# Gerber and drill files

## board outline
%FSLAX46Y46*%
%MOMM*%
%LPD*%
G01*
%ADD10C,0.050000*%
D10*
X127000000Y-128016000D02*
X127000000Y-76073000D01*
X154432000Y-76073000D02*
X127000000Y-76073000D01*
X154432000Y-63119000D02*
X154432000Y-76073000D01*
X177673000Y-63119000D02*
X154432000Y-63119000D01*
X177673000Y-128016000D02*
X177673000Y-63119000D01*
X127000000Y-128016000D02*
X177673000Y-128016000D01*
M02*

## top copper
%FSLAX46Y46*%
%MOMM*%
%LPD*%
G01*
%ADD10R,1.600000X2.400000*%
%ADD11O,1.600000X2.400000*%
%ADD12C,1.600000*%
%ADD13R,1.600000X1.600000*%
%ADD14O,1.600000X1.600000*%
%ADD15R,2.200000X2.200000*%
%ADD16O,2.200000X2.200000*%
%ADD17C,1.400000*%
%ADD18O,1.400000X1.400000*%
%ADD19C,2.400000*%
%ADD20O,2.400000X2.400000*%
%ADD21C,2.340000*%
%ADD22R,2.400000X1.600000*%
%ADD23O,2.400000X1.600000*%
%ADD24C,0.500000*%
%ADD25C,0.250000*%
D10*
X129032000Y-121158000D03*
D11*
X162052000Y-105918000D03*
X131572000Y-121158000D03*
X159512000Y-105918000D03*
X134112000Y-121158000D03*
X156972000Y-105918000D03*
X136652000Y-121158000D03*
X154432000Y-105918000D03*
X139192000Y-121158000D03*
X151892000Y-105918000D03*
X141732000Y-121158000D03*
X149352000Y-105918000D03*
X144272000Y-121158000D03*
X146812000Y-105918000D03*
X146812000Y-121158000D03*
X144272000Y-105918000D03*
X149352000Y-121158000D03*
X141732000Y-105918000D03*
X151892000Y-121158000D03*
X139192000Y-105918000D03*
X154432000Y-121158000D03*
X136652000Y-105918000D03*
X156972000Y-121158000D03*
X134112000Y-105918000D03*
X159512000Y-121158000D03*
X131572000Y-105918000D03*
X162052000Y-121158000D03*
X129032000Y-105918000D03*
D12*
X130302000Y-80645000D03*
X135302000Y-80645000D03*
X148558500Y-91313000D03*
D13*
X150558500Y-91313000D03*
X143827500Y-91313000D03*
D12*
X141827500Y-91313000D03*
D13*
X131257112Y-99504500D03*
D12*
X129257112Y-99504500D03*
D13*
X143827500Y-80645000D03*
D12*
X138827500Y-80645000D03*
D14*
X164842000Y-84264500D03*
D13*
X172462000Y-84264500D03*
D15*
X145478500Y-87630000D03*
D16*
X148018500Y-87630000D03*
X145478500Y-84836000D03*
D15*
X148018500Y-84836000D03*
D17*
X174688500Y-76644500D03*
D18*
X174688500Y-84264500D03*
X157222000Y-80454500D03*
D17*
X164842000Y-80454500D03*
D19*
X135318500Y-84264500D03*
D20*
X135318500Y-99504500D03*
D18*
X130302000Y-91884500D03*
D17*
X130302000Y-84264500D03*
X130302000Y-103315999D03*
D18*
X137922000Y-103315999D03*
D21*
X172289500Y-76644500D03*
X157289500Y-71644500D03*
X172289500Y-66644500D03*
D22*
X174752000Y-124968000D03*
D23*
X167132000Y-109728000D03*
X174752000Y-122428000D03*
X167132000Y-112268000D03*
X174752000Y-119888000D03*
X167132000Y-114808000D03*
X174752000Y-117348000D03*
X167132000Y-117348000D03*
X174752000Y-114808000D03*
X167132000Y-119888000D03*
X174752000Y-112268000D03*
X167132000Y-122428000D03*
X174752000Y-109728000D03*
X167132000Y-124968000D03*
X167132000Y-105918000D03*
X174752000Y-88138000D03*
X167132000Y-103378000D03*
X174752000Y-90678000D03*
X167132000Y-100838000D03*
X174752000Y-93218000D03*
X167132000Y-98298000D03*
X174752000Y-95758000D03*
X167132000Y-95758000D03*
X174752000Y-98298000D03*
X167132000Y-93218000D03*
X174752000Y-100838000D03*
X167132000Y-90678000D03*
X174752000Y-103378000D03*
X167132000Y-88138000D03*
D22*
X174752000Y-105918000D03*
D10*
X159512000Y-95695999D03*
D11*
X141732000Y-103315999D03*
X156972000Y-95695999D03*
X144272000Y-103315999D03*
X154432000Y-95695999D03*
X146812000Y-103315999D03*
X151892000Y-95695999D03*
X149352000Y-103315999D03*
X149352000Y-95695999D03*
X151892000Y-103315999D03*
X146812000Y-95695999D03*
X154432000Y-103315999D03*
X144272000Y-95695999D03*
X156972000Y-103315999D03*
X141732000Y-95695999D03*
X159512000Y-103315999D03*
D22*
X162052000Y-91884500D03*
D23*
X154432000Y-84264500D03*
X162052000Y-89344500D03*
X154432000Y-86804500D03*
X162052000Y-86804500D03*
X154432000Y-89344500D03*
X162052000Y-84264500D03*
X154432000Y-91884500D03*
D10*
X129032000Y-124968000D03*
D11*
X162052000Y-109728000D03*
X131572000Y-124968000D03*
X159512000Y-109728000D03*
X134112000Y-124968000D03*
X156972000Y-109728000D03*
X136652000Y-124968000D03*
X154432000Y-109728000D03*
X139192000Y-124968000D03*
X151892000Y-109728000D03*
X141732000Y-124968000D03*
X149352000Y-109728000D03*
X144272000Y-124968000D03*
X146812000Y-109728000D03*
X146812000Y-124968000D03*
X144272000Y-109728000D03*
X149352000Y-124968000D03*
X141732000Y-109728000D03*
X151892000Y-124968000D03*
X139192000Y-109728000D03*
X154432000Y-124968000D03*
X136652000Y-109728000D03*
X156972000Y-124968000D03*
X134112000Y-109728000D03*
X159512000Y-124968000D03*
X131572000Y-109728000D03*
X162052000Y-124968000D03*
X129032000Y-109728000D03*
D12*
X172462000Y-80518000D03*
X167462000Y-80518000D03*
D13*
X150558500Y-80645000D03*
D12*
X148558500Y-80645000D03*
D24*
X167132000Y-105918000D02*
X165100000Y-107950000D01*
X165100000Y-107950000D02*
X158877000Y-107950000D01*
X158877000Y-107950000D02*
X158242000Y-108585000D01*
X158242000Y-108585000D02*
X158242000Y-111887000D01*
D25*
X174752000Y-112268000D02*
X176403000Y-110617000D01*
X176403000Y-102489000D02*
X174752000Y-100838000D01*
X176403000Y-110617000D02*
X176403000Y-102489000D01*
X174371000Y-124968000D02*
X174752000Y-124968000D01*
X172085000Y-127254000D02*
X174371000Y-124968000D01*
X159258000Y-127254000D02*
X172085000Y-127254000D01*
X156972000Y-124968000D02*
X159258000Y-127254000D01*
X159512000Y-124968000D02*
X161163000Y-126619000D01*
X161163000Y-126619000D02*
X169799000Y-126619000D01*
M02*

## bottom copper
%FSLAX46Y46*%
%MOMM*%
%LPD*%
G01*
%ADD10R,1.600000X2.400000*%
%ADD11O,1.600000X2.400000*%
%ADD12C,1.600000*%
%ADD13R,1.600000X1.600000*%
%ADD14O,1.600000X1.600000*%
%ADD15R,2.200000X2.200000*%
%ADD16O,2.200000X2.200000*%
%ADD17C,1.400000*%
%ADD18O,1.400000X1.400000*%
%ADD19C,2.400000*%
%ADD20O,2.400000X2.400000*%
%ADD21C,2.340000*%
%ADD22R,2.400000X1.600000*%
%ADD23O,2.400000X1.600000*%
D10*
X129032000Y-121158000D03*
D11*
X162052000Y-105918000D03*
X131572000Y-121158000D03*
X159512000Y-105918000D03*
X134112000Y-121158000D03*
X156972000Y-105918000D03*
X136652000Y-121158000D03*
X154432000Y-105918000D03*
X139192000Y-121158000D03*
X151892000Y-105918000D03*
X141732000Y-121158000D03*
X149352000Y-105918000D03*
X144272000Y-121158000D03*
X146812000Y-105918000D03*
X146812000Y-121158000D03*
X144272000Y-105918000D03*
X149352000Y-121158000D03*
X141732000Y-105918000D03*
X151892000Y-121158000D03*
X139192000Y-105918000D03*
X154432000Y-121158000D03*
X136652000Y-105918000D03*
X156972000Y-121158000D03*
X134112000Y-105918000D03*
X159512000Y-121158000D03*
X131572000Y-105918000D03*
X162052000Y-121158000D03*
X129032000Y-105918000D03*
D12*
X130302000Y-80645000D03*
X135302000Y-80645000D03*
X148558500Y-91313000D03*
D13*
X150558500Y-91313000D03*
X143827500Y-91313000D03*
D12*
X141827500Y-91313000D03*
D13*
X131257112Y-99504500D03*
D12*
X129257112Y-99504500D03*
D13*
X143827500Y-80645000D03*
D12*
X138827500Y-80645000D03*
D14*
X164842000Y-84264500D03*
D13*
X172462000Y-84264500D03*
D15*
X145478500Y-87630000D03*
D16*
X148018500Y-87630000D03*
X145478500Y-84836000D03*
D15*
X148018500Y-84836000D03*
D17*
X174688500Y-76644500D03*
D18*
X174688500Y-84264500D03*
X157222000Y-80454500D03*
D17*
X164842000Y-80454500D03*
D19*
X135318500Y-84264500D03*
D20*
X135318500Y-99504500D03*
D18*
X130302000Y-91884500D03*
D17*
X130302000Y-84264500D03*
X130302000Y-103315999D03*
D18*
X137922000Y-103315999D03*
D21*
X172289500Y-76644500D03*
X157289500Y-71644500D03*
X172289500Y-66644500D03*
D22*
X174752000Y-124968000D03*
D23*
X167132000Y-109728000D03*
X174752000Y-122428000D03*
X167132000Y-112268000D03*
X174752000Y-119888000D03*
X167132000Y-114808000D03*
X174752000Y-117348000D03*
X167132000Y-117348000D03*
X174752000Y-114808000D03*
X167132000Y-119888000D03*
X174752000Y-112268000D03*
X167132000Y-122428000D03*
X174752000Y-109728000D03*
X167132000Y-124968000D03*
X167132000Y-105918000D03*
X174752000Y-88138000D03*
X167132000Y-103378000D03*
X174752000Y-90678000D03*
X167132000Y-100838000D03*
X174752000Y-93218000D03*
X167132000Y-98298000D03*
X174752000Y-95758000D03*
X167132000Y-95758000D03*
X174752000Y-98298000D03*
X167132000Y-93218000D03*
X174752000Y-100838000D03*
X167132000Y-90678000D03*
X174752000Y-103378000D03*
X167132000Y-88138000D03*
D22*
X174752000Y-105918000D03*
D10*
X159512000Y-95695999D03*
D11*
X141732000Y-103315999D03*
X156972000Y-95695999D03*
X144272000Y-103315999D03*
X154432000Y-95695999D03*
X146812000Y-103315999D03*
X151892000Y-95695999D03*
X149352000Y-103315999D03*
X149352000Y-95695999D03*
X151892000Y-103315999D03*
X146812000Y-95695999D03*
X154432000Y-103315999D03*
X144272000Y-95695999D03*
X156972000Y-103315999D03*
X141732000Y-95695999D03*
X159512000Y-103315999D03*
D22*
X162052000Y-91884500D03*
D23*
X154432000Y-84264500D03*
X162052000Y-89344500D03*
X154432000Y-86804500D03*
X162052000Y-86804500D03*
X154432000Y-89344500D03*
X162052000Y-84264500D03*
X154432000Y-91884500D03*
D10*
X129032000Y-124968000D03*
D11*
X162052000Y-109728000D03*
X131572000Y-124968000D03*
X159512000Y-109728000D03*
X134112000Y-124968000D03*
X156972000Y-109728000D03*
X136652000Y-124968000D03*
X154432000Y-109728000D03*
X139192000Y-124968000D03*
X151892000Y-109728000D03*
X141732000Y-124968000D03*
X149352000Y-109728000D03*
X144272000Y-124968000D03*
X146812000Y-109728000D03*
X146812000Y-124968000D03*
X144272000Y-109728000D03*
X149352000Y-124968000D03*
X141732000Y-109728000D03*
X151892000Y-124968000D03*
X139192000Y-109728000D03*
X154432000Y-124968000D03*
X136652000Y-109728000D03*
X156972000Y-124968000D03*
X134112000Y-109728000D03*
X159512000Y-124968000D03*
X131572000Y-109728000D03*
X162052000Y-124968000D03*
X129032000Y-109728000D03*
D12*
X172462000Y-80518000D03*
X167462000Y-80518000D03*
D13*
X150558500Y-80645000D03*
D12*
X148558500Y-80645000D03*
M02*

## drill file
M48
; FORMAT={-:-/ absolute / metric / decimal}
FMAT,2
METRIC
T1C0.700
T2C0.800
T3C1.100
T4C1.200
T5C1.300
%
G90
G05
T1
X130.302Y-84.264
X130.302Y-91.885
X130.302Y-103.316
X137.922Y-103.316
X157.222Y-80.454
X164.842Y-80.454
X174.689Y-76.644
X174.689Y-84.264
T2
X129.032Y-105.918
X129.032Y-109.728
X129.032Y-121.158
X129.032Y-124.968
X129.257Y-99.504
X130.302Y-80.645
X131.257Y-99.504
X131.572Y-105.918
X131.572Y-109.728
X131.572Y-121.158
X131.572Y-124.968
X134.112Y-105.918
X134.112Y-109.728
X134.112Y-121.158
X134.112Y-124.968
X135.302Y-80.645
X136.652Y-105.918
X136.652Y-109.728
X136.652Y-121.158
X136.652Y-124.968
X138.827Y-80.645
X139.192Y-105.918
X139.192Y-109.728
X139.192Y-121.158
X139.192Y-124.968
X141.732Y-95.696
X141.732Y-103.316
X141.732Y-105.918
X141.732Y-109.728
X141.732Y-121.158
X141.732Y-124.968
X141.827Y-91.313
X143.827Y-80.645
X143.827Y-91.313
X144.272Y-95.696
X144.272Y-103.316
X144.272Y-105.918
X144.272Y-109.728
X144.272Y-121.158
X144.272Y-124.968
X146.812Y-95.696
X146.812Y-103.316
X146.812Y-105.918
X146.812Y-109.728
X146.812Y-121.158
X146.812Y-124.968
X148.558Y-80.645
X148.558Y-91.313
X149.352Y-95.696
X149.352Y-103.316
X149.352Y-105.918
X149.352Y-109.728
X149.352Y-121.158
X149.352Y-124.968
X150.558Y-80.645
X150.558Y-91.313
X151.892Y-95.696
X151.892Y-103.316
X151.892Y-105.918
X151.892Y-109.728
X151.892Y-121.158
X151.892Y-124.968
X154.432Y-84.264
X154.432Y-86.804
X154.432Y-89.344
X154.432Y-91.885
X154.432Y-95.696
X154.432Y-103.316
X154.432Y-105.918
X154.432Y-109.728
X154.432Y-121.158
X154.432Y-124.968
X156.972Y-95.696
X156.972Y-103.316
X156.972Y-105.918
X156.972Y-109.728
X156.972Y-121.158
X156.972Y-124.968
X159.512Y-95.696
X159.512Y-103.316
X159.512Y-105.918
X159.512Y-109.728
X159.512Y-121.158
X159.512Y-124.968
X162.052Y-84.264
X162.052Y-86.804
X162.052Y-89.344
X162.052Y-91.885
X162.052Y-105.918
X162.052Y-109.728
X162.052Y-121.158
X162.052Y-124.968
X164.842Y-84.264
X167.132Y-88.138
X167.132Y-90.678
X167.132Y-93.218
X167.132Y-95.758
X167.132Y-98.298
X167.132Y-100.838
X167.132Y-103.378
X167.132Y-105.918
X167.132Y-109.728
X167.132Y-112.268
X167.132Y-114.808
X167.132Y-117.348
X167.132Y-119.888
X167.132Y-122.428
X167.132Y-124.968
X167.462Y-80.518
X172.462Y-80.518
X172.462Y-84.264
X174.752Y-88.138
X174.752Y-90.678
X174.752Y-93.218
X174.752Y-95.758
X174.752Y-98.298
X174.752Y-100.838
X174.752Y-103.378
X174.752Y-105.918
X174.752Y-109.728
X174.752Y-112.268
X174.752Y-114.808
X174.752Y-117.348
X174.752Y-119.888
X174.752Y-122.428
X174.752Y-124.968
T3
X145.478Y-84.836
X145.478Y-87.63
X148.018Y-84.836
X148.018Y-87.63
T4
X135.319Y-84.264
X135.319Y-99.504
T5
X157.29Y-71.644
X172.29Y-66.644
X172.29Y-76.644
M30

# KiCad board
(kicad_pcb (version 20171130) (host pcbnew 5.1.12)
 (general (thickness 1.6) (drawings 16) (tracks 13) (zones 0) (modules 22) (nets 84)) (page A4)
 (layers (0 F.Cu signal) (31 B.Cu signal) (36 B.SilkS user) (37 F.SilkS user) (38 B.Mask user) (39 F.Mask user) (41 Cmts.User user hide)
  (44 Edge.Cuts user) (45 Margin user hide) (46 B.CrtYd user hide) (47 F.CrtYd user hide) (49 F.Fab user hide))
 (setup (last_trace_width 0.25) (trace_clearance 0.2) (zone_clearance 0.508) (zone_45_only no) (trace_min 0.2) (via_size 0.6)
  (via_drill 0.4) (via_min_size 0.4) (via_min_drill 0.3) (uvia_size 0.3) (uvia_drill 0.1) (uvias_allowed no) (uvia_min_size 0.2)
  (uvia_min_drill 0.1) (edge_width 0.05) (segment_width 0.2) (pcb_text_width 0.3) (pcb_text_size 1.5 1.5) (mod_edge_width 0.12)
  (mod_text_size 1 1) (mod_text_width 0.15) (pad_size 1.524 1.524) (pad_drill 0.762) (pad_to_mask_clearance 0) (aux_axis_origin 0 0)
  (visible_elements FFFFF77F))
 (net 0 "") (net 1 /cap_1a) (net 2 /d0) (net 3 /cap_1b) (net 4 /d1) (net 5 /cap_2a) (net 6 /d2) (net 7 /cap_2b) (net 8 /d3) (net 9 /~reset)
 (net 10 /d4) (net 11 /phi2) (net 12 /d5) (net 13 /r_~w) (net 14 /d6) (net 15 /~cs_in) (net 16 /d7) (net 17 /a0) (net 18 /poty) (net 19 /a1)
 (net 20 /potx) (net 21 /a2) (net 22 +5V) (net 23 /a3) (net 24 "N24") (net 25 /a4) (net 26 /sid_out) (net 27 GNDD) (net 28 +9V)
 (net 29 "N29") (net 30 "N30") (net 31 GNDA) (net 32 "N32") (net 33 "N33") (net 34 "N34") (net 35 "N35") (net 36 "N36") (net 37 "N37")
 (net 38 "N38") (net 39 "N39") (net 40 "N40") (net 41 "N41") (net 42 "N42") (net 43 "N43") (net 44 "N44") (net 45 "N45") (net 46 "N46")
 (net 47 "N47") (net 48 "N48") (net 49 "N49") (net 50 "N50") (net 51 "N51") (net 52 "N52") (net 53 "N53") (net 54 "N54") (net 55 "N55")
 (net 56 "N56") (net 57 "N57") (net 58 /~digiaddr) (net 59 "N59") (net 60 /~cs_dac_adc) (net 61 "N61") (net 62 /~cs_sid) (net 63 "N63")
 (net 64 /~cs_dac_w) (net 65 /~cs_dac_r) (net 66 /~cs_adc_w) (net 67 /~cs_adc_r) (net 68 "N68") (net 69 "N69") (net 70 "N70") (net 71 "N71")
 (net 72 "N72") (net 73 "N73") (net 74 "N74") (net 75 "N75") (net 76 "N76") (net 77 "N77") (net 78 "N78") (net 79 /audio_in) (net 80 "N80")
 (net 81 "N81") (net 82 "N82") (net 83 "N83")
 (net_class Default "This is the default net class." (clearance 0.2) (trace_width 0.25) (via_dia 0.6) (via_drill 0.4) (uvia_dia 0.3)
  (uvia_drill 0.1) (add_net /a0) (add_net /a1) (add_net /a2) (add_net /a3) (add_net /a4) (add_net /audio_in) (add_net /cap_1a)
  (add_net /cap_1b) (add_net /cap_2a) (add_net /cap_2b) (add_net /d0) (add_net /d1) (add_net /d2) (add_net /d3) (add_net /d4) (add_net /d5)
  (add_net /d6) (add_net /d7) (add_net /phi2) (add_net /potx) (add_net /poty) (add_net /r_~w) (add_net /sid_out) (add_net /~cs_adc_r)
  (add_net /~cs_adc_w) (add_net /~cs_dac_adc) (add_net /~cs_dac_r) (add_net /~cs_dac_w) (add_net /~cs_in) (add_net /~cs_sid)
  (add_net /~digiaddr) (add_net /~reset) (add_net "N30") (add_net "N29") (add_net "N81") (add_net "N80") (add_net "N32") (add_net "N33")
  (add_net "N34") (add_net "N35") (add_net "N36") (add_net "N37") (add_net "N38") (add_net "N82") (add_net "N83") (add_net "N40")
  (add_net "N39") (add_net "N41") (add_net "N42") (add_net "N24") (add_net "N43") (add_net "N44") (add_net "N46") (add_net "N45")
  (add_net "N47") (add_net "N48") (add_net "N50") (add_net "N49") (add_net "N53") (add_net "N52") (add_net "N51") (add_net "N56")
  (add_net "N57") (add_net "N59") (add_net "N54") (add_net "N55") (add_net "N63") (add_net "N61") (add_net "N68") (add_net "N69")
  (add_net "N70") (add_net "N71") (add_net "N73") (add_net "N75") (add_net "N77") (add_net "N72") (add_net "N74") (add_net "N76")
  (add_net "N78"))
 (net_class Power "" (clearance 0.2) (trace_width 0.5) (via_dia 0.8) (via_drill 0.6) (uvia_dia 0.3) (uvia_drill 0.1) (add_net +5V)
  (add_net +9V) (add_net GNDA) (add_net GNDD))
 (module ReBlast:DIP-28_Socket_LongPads (layer F.Cu) (at 129.032 121.158 90)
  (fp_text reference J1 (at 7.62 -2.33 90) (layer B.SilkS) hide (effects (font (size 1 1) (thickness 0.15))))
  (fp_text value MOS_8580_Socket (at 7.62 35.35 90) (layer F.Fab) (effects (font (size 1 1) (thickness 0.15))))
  (pad 1 thru_hole rect (at 0 0 90) (size 2.4 1.6) (drill 0.8) (layers *.Cu *.Mask) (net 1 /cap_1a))
  (pad 15 thru_hole oval (at 15.24 33.02 90) (size 2.4 1.6) (drill 0.8) (layers *.Cu *.Mask) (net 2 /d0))
  (pad 2 thru_hole oval (at 0 2.54 90) (size 2.4 1.6) (drill 0.8) (layers *.Cu *.Mask) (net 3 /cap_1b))
  (pad 16 thru_hole oval (at 15.24 30.48 90) (size 2.4 1.6) (drill 0.8) (layers *.Cu *.Mask) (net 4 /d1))
  (pad 3 thru_hole oval (at 0 5.08 90) (size 2.4 1.6) (drill 0.8) (layers *.Cu *.Mask) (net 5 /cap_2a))
  (pad 17 thru_hole oval (at 15.24 27.94 90) (size 2.4 1.6) (drill 0.8) (layers *.Cu *.Mask) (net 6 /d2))
  (pad 4 thru_hole oval (at 0 7.62 90) (size 2.4 1.6) (drill 0.8) (layers *.Cu *.Mask) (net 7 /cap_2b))
  (pad 18 thru_hole oval (at 15.24 25.4 90) (size 2.4 1.6) (drill 0.8) (layers *.Cu *.Mask) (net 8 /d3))
  (pad 5 thru_hole oval (at 0 10.16 90) (size 2.4 1.6) (drill 0.8) (layers *.Cu *.Mask) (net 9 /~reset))
  (pad 19 thru_hole oval (at 15.24 22.86 90) (size 2.4 1.6) (drill 0.8) (layers *.Cu *.Mask) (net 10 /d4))
  (pad 6 thru_hole oval (at 0 12.7 90) (size 2.4 1.6) (drill 0.8) (layers *.Cu *.Mask) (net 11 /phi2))
  (pad 20 thru_hole oval (at 15.24 20.32 90) (size 2.4 1.6) (drill 0.8) (layers *.Cu *.Mask) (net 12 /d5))
  (pad 7 thru_hole oval (at 0 15.24 90) (size 2.4 1.6) (drill 0.8) (layers *.Cu *.Mask) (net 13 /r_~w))
  (pad 21 thru_hole oval (at 15.24 17.78 90) (size 2.4 1.6) (drill 0.8) (layers *.Cu *.Mask) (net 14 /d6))
  (pad 8 thru_hole oval (at 0 17.78 90) (size 2.4 1.6) (drill 0.8) (layers *.Cu *.Mask) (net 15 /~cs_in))
  (pad 22 thru_hole oval (at 15.24 15.24 90) (size 2.4 1.6) (drill 0.8) (layers *.Cu *.Mask) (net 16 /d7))
  (pad 9 thru_hole oval (at 0 20.32 90) (size 2.4 1.6) (drill 0.8) (layers *.Cu *.Mask) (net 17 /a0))
  (pad 23 thru_hole oval (at 15.24 12.7 90) (size 2.4 1.6) (drill 0.8) (layers *.Cu *.Mask) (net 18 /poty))
  (pad 10 thru_hole oval (at 0 22.86 90) (size 2.4 1.6) (drill 0.8) (layers *.Cu *.Mask) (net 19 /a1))
  (pad 24 thru_hole oval (at 15.24 10.16 90) (size 2.4 1.6) (drill 0.8) (layers *.Cu *.Mask) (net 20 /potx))
  (pad 11 thru_hole oval (at 0 25.4 90) (size 2.4 1.6) (drill 0.8) (layers *.Cu *.Mask) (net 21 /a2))
  (pad 25 thru_hole oval (at 15.24 7.62 90) (size 2.4 1.6) (drill 0.8) (layers *.Cu *.Mask) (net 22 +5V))
  (pad 12 thru_hole oval (at 0 27.94 90) (size 2.4 1.6) (drill 0.8) (layers *.Cu *.Mask) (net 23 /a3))
  (pad 26 thru_hole oval (at 15.24 5.08 90) (size 2.4 1.6) (drill 0.8) (layers *.Cu *.Mask) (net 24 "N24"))
  (pad 13 thru_hole oval (at 0 30.48 90) (size 2.4 1.6) (drill 0.8) (layers *.Cu *.Mask) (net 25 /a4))
  (pad 27 thru_hole oval (at 15.24 2.54 90) (size 2.4 1.6) (drill 0.8) (layers *.Cu *.Mask) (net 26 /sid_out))
  (pad 14 thru_hole oval (at 0 33.02 90) (size 2.4 1.6) (drill 0.8) (layers *.Cu *.Mask) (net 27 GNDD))
  (pad 28 thru_hole oval (at 15.24 0 90) (size 2.4 1.6) (drill 0.8) (layers *.Cu *.Mask) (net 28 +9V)))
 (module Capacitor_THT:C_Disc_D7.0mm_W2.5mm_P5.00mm (layer F.Cu) (at 135.302 80.645 180)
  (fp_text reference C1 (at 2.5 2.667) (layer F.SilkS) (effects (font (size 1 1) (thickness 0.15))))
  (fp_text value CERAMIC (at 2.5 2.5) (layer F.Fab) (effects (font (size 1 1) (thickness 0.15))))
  (pad 2 thru_hole circle (at 5 0 180) (size 1.6 1.6) (drill 0.8) (layers *.Cu *.Mask) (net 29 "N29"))
  (pad 1 thru_hole circle (at 0 0 180) (size 1.6 1.6) (drill 0.8) (layers *.Cu *.Mask) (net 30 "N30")))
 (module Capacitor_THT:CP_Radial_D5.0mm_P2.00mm (layer F.Cu) (at 150.5585 91.313 180)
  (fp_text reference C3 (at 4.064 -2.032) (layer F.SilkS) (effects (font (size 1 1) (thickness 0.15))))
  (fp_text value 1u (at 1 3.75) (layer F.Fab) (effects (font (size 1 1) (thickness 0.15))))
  (pad 2 thru_hole circle (at 2 0 180) (size 1.6 1.6) (drill 0.8) (layers *.Cu *.Mask) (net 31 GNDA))
  (pad 1 thru_hole rect (at 0 0 180) (size 1.6 1.6) (drill 0.8) (layers *.Cu *.Mask) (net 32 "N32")))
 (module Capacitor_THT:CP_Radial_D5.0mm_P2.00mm (layer F.Cu) (at 143.8275 91.313 180)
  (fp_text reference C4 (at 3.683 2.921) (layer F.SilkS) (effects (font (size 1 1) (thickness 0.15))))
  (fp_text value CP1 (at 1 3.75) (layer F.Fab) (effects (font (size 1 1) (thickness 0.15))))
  (pad 1 thru_hole rect (at 0 0 180) (size 1.6 1.6) (drill 0.8) (layers *.Cu *.Mask) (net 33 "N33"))
  (pad 2 thru_hole circle (at 2 0 180) (size 1.6 1.6) (drill 0.8) (layers *.Cu *.Mask) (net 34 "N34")))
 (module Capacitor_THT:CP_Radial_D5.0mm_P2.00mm (layer F.Cu) (at 131.257112 99.5045 180)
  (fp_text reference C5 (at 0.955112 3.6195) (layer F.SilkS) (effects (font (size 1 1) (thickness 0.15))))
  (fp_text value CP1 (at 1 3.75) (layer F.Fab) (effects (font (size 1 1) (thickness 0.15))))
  (pad 1 thru_hole rect (at 0 0 180) (size 1.6 1.6) (drill 0.8) (layers *.Cu *.Mask) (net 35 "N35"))
  (pad 2 thru_hole circle (at 2 0 180) (size 1.6 1.6) (drill 0.8) (layers *.Cu *.Mask) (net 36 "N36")))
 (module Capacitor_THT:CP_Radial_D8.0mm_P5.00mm (layer F.Cu) (at 143.8275 80.645 180)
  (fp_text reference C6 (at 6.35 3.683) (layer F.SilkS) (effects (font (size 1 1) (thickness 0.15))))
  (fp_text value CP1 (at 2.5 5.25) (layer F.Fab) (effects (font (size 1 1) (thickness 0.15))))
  (pad 1 thru_hole rect (at 0 0 180) (size 1.6 1.6) (drill 0.8) (layers *.Cu *.Mask) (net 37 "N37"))
  (pad 2 thru_hole circle (at 5 0 180) (size 1.6 1.6) (drill 0.8) (layers *.Cu *.Mask) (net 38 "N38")))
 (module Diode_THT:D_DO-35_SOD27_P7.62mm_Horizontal (layer F.Cu) (at 172.462 84.2645 180)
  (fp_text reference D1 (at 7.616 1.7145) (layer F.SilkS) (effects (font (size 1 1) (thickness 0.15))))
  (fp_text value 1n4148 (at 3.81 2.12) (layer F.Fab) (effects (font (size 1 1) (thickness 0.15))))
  (pad 2 thru_hole oval (at 7.62 0 180) (size 1.6 1.6) (drill 0.8) (layers *.Cu *.Mask) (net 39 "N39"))
  (pad 1 thru_hole rect (at 0 0 180) (size 1.6 1.6) (drill 0.8) (layers *.Cu *.Mask) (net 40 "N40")))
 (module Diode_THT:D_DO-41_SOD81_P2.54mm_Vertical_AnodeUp (layer F.Cu) (at 145.4785 87.63)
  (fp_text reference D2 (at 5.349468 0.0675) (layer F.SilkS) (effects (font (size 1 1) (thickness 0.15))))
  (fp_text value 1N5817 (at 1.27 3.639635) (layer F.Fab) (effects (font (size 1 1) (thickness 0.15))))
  (pad 1 thru_hole rect (at 0 0) (size 2.2 2.2) (drill 1.1) (layers *.Cu *.Mask) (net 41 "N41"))
  (pad 2 thru_hole oval (at 2.54 0) (size 2.2 2.2) (drill 1.1) (layers *.Cu *.Mask) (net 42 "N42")))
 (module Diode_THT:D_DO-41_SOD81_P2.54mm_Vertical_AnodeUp (layer F.Cu) (at 148.0185 84.836 180)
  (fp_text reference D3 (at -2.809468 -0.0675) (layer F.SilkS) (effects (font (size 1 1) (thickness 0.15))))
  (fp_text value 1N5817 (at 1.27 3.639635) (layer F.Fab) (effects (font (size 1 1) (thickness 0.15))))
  (pad 2 thru_hole oval (at 2.54 0 180) (size 2.2 2.2) (drill 1.1) (layers *.Cu *.Mask) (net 41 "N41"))
  (pad 1 thru_hole rect (at 0 0 180) (size 2.2 2.2) (drill 1.1) (layers *.Cu *.Mask) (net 27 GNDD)))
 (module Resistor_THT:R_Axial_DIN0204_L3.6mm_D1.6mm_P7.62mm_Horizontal (layer F.Cu) (at 174.6885 76.6445 270)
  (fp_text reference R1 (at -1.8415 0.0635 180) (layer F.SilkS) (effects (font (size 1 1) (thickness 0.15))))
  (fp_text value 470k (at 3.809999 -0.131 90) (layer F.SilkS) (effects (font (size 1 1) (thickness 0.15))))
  (pad 1 thru_hole circle (at 0 0 270) (size 1.4 1.4) (drill 0.7) (layers *.Cu *.Mask) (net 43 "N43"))
  (pad 2 thru_hole oval (at 7.62 0 270) (size 1.4 1.4) (drill 0.7) (layers *.Cu *.Mask) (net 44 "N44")))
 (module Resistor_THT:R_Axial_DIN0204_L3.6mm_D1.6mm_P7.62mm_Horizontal (layer F.Cu) (at 164.842 80.4545 180)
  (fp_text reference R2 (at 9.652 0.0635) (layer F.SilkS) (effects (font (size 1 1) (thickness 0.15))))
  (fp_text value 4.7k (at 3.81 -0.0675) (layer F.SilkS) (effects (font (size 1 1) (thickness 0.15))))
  (pad 2 thru_hole oval (at 7.62 0 180) (size 1.4 1.4) (drill 0.7) (layers *.Cu *.Mask) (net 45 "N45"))
  (pad 1 thru_hole circle (at 0 0 180) (size 1.4 1.4) (drill 0.7) (layers *.Cu *.Mask) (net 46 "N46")))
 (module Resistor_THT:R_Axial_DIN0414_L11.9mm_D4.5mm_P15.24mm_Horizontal (layer F.Cu) (at 135.3185 84.2645 270)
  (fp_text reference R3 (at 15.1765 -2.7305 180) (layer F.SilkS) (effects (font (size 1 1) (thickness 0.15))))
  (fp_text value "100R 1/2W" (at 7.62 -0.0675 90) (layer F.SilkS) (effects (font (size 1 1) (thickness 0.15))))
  (pad 1 thru_hole circle (at 0 0 270) (size 2.4 2.4) (drill 1.2) (layers *.Cu *.Mask) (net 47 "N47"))
  (pad 2 thru_hole oval (at 15.24 0 270) (size 2.4 2.4) (drill 1.2) (layers *.Cu *.Mask) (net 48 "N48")))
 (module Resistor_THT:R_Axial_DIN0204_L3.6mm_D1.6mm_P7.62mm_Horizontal (layer F.Cu) (at 130.302 84.2645 270)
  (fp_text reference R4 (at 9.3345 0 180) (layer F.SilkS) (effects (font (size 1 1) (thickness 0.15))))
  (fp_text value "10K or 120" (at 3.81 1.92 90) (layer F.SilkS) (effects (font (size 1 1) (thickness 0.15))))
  (pad 2 thru_hole oval (at 7.62 0 270) (size 1.4 1.4) (drill 0.7) (layers *.Cu *.Mask) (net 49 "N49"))
  (pad 1 thru_hole circle (at 0 0 270) (size 1.4 1.4) (drill 0.7) (layers *.Cu *.Mask) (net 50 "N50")))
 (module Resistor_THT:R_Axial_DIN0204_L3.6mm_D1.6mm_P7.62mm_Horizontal (layer F.Cu) (at 130.302 103.315999)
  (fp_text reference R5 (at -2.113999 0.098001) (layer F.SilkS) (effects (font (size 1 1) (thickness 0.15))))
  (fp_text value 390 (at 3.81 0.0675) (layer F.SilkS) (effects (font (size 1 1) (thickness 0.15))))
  (pad 1 thru_hole circle (at 0 0) (size 1.4 1.4) (drill 0.7) (layers *.Cu *.Mask) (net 22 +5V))
  (pad 2 thru_hole oval (at 7.62 0) (size 1.4 1.4) (drill 0.7) (layers *.Cu *.Mask) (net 32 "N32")))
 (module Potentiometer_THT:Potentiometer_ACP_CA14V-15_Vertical (layer F.Cu) (at 172.2895 66.6445 180)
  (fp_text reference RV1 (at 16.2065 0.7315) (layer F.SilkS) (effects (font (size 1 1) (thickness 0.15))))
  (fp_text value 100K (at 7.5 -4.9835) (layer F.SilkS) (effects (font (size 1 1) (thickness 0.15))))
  (pad 3 thru_hole circle (at 0 -10 180) (size 2.34 2.34) (drill 1.3) (layers *.Cu *.Mask) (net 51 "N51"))
  (pad 2 thru_hole circle (at 15 -5 180) (size 2.34 2.34) (drill 1.3) (layers *.Cu *.Mask) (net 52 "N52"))
  (pad 1 thru_hole circle (at 0 0 180) (size 2.34 2.34) (drill 1.3) (layers *.Cu *.Mask) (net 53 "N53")))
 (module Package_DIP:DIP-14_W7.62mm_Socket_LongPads (layer F.Cu) (at 174.752 124.968 180)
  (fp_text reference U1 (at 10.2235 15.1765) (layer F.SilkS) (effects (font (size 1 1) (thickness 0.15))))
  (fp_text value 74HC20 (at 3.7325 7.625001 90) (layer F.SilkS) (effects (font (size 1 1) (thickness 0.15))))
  (pad 1 thru_hole rect (at 0 0 180) (size 2.4 1.6) (drill 0.8) (layers *.Cu *.Mask) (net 23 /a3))
  (pad 8 thru_hole oval (at 7.62 15.24 180) (size 2.4 1.6) (drill 0.8) (layers *.Cu *.Mask) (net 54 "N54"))
  (pad 2 thru_hole oval (at 0 2.54 180) (size 2.4 1.6) (drill 0.8) (layers *.Cu *.Mask) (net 21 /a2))
  (pad 9 thru_hole oval (at 7.62 12.7 180) (size 2.4 1.6) (drill 0.8) (layers *.Cu *.Mask) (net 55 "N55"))
  (pad 3 thru_hole oval (at 0 5.08 180) (size 2.4 1.6) (drill 0.8) (layers *.Cu *.Mask))
  (pad 10 thru_hole oval (at 7.62 10.16 180) (size 2.4 1.6) (drill 0.8) (layers *.Cu *.Mask) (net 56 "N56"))
  (pad 4 thru_hole oval (at 0 7.62 180) (size 2.4 1.6) (drill 0.8) (layers *.Cu *.Mask) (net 19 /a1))
  (pad 11 thru_hole oval (at 7.62 7.62 180) (size 2.4 1.6) (drill 0.8) (layers *.Cu *.Mask))
  (pad 5 thru_hole oval (at 0 10.16 180) (size 2.4 1.6) (drill 0.8) (layers *.Cu *.Mask) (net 25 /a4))
  (pad 12 thru_hole oval (at 7.62 5.08 180) (size 2.4 1.6) (drill 0.8) (layers *.Cu *.Mask) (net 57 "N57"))
  (pad 6 thru_hole oval (at 0 12.7 180) (size 2.4 1.6) (drill 0.8) (layers *.Cu *.Mask) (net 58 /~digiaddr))
  (pad 13 thru_hole oval (at 7.62 2.54 180) (size 2.4 1.6) (drill 0.8) (layers *.Cu *.Mask) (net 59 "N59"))
  (pad 7 thru_hole oval (at 0 15.24 180) (size 2.4 1.6) (drill 0.8) (layers *.Cu *.Mask) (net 27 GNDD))
  (pad 14 thru_hole oval (at 7.62 0 180) (size 2.4 1.6) (drill 0.8) (layers *.Cu *.Mask) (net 22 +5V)))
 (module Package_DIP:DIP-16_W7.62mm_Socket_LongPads (layer F.Cu) (at 174.752 105.918 180)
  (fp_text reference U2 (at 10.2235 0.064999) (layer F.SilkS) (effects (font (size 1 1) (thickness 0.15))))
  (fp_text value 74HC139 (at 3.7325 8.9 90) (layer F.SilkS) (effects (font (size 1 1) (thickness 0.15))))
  (pad 16 thru_hole oval (at 7.62 0 180) (size 2.4 1.6) (drill 0.8) (layers *.Cu *.Mask) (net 22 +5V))
  (pad 8 thru_hole oval (at 0 17.78 180) (size 2.4 1.6) (drill 0.8) (layers *.Cu *.Mask) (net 27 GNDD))
  (pad 15 thru_hole oval (at 7.62 2.54 180) (size 2.4 1.6) (drill 0.8) (layers *.Cu *.Mask) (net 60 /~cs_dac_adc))
  (pad 7 thru_hole oval (at 0 15.24 180) (size 2.4 1.6) (drill 0.8) (layers *.Cu *.Mask) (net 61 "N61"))
  (pad 14 thru_hole oval (at 7.62 5.08 180) (size 2.4 1.6) (drill 0.8) (layers *.Cu *.Mask) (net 13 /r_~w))
  (pad 6 thru_hole oval (at 0 12.7 180) (size 2.4 1.6) (drill 0.8) (layers *.Cu *.Mask) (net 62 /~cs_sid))
  (pad 13 thru_hole oval (at 7.62 7.62 180) (size 2.4 1.6) (drill 0.8) (layers *.Cu *.Mask) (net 17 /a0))
  (pad 5 thru_hole oval (at 0 10.16 180) (size 2.4 1.6) (drill 0.8) (layers *.Cu *.Mask) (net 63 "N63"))
  (pad 12 thru_hole oval (at 7.62 10.16 180) (size 2.4 1.6) (drill 0.8) (layers *.Cu *.Mask) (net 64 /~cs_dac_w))
  (pad 4 thru_hole oval (at 0 7.62 180) (size 2.4 1.6) (drill 0.8) (layers *.Cu *.Mask) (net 60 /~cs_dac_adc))
  (pad 11 thru_hole oval (at 7.62 12.7 180) (size 2.4 1.6) (drill 0.8) (layers *.Cu *.Mask) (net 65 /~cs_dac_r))
  (pad 3 thru_hole oval (at 0 5.08 180) (size 2.4 1.6) (drill 0.8) (layers *.Cu *.Mask) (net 58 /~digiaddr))
  (pad 10 thru_hole oval (at 7.62 15.24 180) (size 2.4 1.6) (drill 0.8) (layers *.Cu *.Mask) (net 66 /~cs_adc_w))
  (pad 2 thru_hole oval (at 0 2.54 180) (size 2.4 1.6) (drill 0.8) (layers *.Cu *.Mask) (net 27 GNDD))
  (pad 9 thru_hole oval (at 7.62 17.78 180) (size 2.4 1.6) (drill 0.8) (layers *.Cu *.Mask) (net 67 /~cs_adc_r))
  (pad 1 thru_hole rect (at 0 0 180) (size 2.4 1.6) (drill 0.8) (layers *.Cu *.Mask) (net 15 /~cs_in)))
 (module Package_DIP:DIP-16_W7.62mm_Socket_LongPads (layer F.Cu) (at 159.512 95.695999 270)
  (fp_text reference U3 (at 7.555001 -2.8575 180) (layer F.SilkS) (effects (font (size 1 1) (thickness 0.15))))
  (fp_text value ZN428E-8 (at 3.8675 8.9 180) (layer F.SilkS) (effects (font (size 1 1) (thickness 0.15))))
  (pad 1 thru_hole rect (at 0 0 270) (size 2.4 1.6) (drill 0.8) (layers *.Cu *.Mask) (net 14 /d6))
  (pad 9 thru_hole oval (at 7.62 17.78 270) (size 2.4 1.6) (drill 0.8) (layers *.Cu *.Mask) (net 27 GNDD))
  (pad 2 thru_hole oval (at 0 2.54 270) (size 2.4 1.6) (drill 0.8) (layers *.Cu *.Mask) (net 16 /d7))
  (pad 10 thru_hole oval (at 7.62 15.24 270) (size 2.4 1.6) (drill 0.8) (layers *.Cu *.Mask) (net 22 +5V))
  (pad 3 thru_hole oval (at 0 5.08 270) (size 2.4 1.6) (drill 0.8) (layers *.Cu *.Mask) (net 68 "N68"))
  (pad 11 thru_hole oval (at 7.62 12.7 270) (size 2.4 1.6) (drill 0.8) (layers *.Cu *.Mask) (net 2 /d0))
  (pad 4 thru_hole oval (at 0 7.62 270) (size 2.4 1.6) (drill 0.8) (layers *.Cu *.Mask) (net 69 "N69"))
  (pad 12 thru_hole oval (at 7.62 10.16 270) (size 2.4 1.6) (drill 0.8) (layers *.Cu *.Mask) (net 4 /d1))
  (pad 5 thru_hole oval (at 0 10.16 270) (size 2.4 1.6) (drill 0.8) (layers *.Cu *.Mask) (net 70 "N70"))
  (pad 13 thru_hole oval (at 7.62 7.62 270) (size 2.4 1.6) (drill 0.8) (layers *.Cu *.Mask) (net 6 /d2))
  (pad 6 thru_hole oval (at 0 12.7 270) (size 2.4 1.6) (drill 0.8) (layers *.Cu *.Mask) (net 32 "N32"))
  (pad 14 thru_hole oval (at 7.62 5.08 270) (size 2.4 1.6) (drill 0.8) (layers *.Cu *.Mask) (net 8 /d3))
  (pad 7 thru_hole oval (at 0 15.24 270) (size 2.4 1.6) (drill 0.8) (layers *.Cu *.Mask) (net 32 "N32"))
  (pad 15 thru_hole oval (at 7.62 2.54 270) (size 2.4 1.6) (drill 0.8) (layers *.Cu *.Mask) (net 10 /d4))
  (pad 8 thru_hole oval (at 0 17.78 270) (size 2.4 1.6) (drill 0.8) (layers *.Cu *.Mask) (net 31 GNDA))
  (pad 16 thru_hole oval (at 7.62 0 270) (size 2.4 1.6) (drill 0.8) (layers *.Cu *.Mask) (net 12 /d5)))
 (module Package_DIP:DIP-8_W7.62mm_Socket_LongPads (layer F.Cu) (at 162.052 91.8845 180)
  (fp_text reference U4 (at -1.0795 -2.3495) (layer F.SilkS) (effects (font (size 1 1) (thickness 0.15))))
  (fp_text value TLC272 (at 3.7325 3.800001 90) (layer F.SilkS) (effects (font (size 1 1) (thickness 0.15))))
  (pad 1 thru_hole rect (at 0 0 180) (size 2.4 1.6) (drill 0.8) (layers *.Cu *.Mask) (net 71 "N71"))
  (pad 5 thru_hole oval (at 7.62 7.62 180) (size 2.4 1.6) (drill 0.8) (layers *.Cu *.Mask) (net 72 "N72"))
  (pad 2 thru_hole oval (at 0 2.54 180) (size 2.4 1.6) (drill 0.8) (layers *.Cu *.Mask) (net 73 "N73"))
  (pad 6 thru_hole oval (at 7.62 5.08 180) (size 2.4 1.6) (drill 0.8) (layers *.Cu *.Mask) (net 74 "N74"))
  (pad 3 thru_hole oval (at 0 5.08 180) (size 2.4 1.6) (drill 0.8) (layers *.Cu *.Mask) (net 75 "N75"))
  (pad 7 thru_hole oval (at 7.62 2.54 180) (size 2.4 1.6) (drill 0.8) (layers *.Cu *.Mask) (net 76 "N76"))
  (pad 4 thru_hole oval (at 0 7.62 180) (size 2.4 1.6) (drill 0.8) (layers *.Cu *.Mask) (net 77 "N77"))
  (pad 8 thru_hole oval (at 7.62 0 180) (size 2.4 1.6) (drill 0.8) (layers *.Cu *.Mask) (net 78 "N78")))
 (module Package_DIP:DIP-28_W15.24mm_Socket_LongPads (layer F.Cu) (at 129.032 124.968 90)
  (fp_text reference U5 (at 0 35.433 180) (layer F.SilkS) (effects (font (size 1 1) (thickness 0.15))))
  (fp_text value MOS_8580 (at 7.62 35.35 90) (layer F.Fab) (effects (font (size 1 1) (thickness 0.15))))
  (pad 1 thru_hole rect (at 0 0 90) (size 2.4 1.6) (drill 0.8) (layers *.Cu *.Mask) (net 1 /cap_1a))
  (pad 15 thru_hole oval (at 15.24 33.02 90) (size 2.4 1.6) (drill 0.8) (layers *.Cu *.Mask) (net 2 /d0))
  (pad 2 thru_hole oval (at 0 2.54 90) (size 2.4 1.6) (drill 0.8) (layers *.Cu *.Mask) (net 3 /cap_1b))
  (pad 16 thru_hole oval (at 15.24 30.48 90) (size 2.4 1.6) (drill 0.8) (layers *.Cu *.Mask) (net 4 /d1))
  (pad 3 thru_hole oval (at 0 5.08 90) (size 2.4 1.6) (drill 0.8) (layers *.Cu *.Mask) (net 5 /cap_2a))
  (pad 17 thru_hole oval (at 15.24 27.94 90) (size 2.4 1.6) (drill 0.8) (layers *.Cu *.Mask) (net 6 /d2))
  (pad 4 thru_hole oval (at 0 7.62 90) (size 2.4 1.6) (drill 0.8) (layers *.Cu *.Mask) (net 7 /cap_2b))
  (pad 18 thru_hole oval (at 15.24 25.4 90) (size 2.4 1.6) (drill 0.8) (layers *.Cu *.Mask) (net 8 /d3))
  (pad 5 thru_hole oval (at 0 10.16 90) (size 2.4 1.6) (drill 0.8) (layers *.Cu *.Mask) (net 9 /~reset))
  (pad 19 thru_hole oval (at 15.24 22.86 90) (size 2.4 1.6) (drill 0.8) (layers *.Cu *.Mask) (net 10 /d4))
  (pad 6 thru_hole oval (at 0 12.7 90) (size 2.4 1.6) (drill 0.8) (layers *.Cu *.Mask) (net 11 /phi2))
  (pad 20 thru_hole oval (at 15.24 20.32 90) (size 2.4 1.6) (drill 0.8) (layers *.Cu *.Mask) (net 12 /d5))
  (pad 7 thru_hole oval (at 0 15.24 90) (size 2.4 1.6) (drill 0.8) (layers *.Cu *.Mask) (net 13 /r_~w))
  (pad 21 thru_hole oval (at 15.24 17.78 90) (size 2.4 1.6) (drill 0.8) (layers *.Cu *.Mask) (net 14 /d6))
  (pad 8 thru_hole oval (at 0 17.78 90) (size 2.4 1.6) (drill 0.8) (layers *.Cu *.Mask) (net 62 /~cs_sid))
  (pad 22 thru_hole oval (at 15.24 15.24 90) (size 2.4 1.6) (drill 0.8) (layers *.Cu *.Mask) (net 16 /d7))
  (pad 9 thru_hole oval (at 0 20.32 90) (size 2.4 1.6) (drill 0.8) (layers *.Cu *.Mask) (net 17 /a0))
  (pad 23 thru_hole oval (at 15.24 12.7 90) (size 2.4 1.6) (drill 0.8) (layers *.Cu *.Mask) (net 18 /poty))
  (pad 10 thru_hole oval (at 0 22.86 90) (size 2.4 1.6) (drill 0.8) (layers *.Cu *.Mask) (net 19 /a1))
  (pad 24 thru_hole oval (at 15.24 10.16 90) (size 2.4 1.6) (drill 0.8) (layers *.Cu *.Mask) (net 20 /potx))
  (pad 11 thru_hole oval (at 0 25.4 90) (size 2.4 1.6) (drill 0.8) (layers *.Cu *.Mask) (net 21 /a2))
  (pad 25 thru_hole oval (at 15.24 7.62 90) (size 2.4 1.6) (drill 0.8) (layers *.Cu *.Mask) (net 22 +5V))
  (pad 12 thru_hole oval (at 0 27.94 90) (size 2.4 1.6) (drill 0.8) (layers *.Cu *.Mask) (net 23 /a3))
  (pad 26 thru_hole oval (at 15.24 5.08 90) (size 2.4 1.6) (drill 0.8) (layers *.Cu *.Mask) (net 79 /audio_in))
  (pad 13 thru_hole oval (at 0 30.48 90) (size 2.4 1.6) (drill 0.8) (layers *.Cu *.Mask) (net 25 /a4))
  (pad 27 thru_hole oval (at 15.24 2.54 90) (size 2.4 1.6) (drill 0.8) (layers *.Cu *.Mask) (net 26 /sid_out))
  (pad 14 thru_hole oval (at 0 33.02 90) (size 2.4 1.6) (drill 0.8) (layers *.Cu *.Mask) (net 27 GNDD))
  (pad 28 thru_hole oval (at 15.24 0 90) (size 2.4 1.6) (drill 0.8) (layers *.Cu *.Mask) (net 28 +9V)))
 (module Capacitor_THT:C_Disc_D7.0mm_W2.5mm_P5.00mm (layer F.Cu) (at 167.462 80.518)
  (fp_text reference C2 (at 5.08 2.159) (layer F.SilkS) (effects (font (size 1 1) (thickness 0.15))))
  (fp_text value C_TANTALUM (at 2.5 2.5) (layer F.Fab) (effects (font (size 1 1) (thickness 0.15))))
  (pad 2 thru_hole circle (at 5 0) (size 1.6 1.6) (drill 0.8) (layers *.Cu *.Mask) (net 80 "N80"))
  (pad 1 thru_hole circle (at 0 0) (size 1.6 1.6) (drill 0.8) (layers *.Cu *.Mask) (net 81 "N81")))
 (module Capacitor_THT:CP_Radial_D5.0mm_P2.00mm (layer F.Cu) (at 150.5585 80.645 180)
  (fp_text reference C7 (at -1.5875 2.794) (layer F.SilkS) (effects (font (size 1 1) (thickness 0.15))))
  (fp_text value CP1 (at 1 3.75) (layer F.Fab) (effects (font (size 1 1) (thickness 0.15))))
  (pad 1 thru_hole rect (at 0 0 180) (size 1.6 1.6) (drill 0.8) (layers *.Cu *.Mask) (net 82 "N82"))
  (pad 2 thru_hole circle (at 2 0 180) (size 1.6 1.6) (drill 0.8) (layers *.Cu *.Mask) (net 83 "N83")))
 (gr_line (start 127 128.016) (end 127 76.073) (layer Edge.Cuts) (width 0.05))
 (gr_line (start 154.432 76.073) (end 127 76.073) (layer Edge.Cuts) (width 0.05))
 (gr_line (start 154.432 63.119) (end 154.432 76.073) (layer Edge.Cuts) (width 0.05))
 (gr_line (start 177.673 63.119) (end 154.432 63.119) (layer Edge.Cuts) (width 0.05))
 (gr_line (start 177.673 128.016) (end 177.673 63.119) (layer Edge.Cuts) (width 0.05))
 (gr_line (start 127 128.016) (end 177.673 128.016) (layer Edge.Cuts) (width 0.05))
 (segment (start 167.132 105.918) (end 165.1 107.95) (width 0.5) (layer F.Cu) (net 22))
 (segment (start 165.1 107.95) (end 158.877 107.95) (width 0.5) (layer F.Cu) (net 22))
 (segment (start 158.877 107.95) (end 158.242 108.585) (width 0.5) (layer F.Cu) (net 22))
 (segment (start 158.242 108.585) (end 158.242 111.887) (width 0.5) (layer F.Cu) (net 22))
 (segment (start 174.752 112.268) (end 176.403 110.617) (width 0.25) (layer F.Cu) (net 58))
 (segment (start 176.403 102.489) (end 174.752 100.838) (width 0.25) (layer F.Cu) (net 58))
 (segment (start 176.403 110.617) (end 176.403 102.489) (width 0.25) (layer F.Cu) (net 58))
 (segment (start 174.371 124.968) (end 174.752 124.968) (width 0.25) (layer F.Cu) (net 23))
 (segment (start 172.085 127.254) (end 174.371 124.968) (width 0.25) (layer F.Cu) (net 23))
 (segment (start 159.258 127.254) (end 172.085 127.254) (width 0.25) (layer F.Cu) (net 23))
 (segment (start 156.972 124.968) (end 159.258 127.254) (width 0.25) (layer F.Cu) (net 23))
 (segment (start 159.512 124.968) (end 161.163 126.619) (width 0.25) (layer F.Cu) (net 25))
 (segment (start 161.163 126.619) (end 169.799 126.619) (width 0.25) (layer F.Cu) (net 25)))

